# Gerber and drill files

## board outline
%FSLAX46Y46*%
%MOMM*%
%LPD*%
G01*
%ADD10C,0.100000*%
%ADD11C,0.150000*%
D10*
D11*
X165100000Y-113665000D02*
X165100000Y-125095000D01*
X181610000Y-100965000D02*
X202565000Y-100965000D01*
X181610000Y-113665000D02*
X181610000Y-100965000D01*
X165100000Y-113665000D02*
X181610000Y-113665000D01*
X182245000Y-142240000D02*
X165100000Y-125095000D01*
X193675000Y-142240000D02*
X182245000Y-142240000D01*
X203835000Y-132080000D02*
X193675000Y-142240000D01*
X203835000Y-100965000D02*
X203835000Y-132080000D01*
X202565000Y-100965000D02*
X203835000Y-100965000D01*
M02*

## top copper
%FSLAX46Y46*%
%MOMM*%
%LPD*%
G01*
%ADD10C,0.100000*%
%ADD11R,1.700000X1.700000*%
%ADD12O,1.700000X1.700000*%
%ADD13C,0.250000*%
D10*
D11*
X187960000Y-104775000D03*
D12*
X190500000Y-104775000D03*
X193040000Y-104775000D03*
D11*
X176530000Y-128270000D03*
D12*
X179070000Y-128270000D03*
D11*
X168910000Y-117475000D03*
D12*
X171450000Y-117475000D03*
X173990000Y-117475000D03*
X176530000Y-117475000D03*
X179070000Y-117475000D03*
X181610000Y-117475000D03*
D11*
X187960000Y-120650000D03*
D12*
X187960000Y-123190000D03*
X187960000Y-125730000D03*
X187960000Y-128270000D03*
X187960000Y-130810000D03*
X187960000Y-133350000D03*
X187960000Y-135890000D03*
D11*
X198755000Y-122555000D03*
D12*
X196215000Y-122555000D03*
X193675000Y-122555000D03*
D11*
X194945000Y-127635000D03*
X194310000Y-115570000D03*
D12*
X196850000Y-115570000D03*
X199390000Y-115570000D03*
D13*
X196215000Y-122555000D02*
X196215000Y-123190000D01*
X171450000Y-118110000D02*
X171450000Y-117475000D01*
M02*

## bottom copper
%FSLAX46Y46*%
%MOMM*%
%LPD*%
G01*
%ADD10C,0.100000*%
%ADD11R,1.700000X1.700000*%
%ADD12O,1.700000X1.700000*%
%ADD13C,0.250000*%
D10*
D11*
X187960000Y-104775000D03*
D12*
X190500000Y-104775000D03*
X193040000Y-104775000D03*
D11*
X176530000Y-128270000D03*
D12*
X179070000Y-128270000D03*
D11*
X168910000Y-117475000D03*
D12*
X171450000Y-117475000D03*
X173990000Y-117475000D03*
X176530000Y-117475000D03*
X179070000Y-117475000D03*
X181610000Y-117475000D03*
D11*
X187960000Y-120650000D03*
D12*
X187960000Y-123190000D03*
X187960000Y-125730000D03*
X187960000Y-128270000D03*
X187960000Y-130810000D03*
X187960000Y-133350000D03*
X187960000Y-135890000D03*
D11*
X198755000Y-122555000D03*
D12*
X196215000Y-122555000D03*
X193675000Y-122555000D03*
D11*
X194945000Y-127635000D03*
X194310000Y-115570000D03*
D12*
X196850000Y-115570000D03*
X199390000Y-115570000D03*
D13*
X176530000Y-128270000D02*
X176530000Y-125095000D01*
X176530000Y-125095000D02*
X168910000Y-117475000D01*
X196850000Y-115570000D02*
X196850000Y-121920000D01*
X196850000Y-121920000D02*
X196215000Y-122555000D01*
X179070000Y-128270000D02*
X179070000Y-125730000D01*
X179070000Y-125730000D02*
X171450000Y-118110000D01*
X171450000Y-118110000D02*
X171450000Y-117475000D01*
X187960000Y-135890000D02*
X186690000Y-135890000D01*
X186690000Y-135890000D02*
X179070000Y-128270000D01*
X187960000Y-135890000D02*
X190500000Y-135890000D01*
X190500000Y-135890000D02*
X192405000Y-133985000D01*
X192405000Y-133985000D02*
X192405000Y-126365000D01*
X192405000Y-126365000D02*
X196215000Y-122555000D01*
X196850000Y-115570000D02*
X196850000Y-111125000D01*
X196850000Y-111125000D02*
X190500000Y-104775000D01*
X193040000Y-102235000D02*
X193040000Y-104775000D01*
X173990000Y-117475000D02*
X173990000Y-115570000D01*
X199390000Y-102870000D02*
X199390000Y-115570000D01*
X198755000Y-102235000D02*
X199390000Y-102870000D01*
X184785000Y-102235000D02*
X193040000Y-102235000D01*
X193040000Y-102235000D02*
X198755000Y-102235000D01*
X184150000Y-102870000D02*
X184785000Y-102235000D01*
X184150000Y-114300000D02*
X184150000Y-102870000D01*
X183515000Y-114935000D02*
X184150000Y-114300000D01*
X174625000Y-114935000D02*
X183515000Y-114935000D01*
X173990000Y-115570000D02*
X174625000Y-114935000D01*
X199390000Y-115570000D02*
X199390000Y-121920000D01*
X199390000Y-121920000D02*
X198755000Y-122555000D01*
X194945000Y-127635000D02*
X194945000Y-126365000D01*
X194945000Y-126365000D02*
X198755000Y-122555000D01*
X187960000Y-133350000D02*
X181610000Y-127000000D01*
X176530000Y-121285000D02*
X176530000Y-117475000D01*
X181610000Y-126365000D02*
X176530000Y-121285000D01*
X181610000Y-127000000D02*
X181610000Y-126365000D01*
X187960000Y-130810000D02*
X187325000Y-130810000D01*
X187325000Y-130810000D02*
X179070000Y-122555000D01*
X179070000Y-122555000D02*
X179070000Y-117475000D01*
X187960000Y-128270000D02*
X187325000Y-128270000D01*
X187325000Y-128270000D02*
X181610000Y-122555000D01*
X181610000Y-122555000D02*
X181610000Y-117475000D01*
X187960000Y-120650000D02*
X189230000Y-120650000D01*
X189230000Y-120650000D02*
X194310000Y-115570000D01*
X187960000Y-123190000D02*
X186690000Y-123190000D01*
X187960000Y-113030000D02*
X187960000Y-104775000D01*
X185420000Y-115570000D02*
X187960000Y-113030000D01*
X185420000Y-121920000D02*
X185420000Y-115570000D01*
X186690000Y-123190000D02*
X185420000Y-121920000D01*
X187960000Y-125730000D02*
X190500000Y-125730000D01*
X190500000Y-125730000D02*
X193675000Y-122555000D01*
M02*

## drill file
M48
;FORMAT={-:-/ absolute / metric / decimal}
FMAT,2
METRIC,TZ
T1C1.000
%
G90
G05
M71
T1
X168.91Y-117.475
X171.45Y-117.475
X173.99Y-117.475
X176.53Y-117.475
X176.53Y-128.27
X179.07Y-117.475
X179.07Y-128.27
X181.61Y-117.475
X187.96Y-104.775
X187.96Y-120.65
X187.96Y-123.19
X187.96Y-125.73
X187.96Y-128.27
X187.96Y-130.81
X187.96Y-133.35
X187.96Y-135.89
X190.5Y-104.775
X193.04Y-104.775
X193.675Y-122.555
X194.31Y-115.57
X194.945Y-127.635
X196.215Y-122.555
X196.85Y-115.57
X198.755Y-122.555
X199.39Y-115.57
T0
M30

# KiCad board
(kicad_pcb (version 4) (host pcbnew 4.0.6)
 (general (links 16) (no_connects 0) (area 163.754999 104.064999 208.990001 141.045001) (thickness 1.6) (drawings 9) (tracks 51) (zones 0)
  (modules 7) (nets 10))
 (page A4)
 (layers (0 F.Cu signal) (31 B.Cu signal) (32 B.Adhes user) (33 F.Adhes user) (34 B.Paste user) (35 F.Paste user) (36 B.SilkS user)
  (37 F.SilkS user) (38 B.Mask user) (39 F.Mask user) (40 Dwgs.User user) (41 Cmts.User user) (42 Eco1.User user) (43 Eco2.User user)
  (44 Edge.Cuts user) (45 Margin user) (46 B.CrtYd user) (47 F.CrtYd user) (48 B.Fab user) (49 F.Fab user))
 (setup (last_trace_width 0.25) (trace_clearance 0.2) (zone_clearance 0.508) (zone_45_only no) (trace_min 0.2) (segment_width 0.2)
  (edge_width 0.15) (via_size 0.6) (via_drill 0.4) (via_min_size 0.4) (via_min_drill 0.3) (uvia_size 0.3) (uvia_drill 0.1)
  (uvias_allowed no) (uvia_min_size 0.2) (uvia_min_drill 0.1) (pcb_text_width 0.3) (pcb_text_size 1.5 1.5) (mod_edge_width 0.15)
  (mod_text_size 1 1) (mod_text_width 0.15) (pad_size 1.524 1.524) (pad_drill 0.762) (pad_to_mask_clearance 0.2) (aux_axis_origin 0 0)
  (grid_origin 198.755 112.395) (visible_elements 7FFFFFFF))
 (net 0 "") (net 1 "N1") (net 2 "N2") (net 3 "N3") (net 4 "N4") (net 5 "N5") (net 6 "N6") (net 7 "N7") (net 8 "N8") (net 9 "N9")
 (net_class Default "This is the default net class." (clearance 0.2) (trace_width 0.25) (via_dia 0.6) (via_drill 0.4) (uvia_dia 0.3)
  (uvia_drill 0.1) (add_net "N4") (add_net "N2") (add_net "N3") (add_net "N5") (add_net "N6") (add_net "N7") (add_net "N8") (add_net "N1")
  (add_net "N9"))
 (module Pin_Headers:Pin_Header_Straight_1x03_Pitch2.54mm (layer F.Cu) (at 187.96 104.775 90)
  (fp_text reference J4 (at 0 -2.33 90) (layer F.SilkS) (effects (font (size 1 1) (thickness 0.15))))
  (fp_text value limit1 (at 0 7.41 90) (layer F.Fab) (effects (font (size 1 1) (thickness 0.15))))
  (pad 1 thru_hole rect (at 0 0 90) (size 1.7 1.7) (drill 1) (layers *.Cu *.Mask) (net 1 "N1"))
  (pad 2 thru_hole oval (at 0 2.54 90) (size 1.7 1.7) (drill 1) (layers *.Cu *.Mask) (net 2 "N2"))
  (pad 3 thru_hole oval (at 0 5.08 90) (size 1.7 1.7) (drill 1) (layers *.Cu *.Mask) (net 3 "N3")))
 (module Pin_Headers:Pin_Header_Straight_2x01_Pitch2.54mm (layer F.Cu) (at 176.53 128.27)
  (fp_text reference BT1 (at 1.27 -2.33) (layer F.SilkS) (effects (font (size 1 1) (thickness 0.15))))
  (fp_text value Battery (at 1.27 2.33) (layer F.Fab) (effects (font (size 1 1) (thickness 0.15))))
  (pad 1 thru_hole rect (at 0 0) (size 1.7 1.7) (drill 1) (layers *.Cu *.Mask) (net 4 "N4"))
  (pad 2 thru_hole oval (at 2.54 0) (size 1.7 1.7) (drill 1) (layers *.Cu *.Mask) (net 2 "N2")))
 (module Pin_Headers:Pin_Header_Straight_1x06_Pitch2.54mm (layer F.Cu) (at 168.91 117.475 90)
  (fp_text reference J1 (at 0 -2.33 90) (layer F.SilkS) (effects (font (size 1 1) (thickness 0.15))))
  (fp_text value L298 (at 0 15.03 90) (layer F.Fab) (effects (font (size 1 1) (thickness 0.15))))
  (pad 1 thru_hole rect (at 0 0 90) (size 1.7 1.7) (drill 1) (layers *.Cu *.Mask) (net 4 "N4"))
  (pad 2 thru_hole oval (at 0 2.54 90) (size 1.7 1.7) (drill 1) (layers *.Cu *.Mask) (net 2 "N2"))
  (pad 3 thru_hole oval (at 0 5.08 90) (size 1.7 1.7) (drill 1) (layers *.Cu *.Mask) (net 3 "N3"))
  (pad 4 thru_hole oval (at 0 7.62 90) (size 1.7 1.7) (drill 1) (layers *.Cu *.Mask) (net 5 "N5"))
  (pad 5 thru_hole oval (at 0 10.16 90) (size 1.7 1.7) (drill 1) (layers *.Cu *.Mask) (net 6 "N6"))
  (pad 6 thru_hole oval (at 0 12.7 90) (size 1.7 1.7) (drill 1) (layers *.Cu *.Mask) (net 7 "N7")))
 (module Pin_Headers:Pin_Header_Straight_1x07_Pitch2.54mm (layer F.Cu) (at 187.96 120.65)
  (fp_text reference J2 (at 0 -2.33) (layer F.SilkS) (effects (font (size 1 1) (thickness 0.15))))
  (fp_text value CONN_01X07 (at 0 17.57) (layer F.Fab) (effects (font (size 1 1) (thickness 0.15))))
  (pad 1 thru_hole rect (at 0 0) (size 1.7 1.7) (drill 1) (layers *.Cu *.Mask) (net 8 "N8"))
  (pad 2 thru_hole oval (at 0 2.54) (size 1.7 1.7) (drill 1) (layers *.Cu *.Mask) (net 1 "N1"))
  (pad 3 thru_hole oval (at 0 5.08) (size 1.7 1.7) (drill 1) (layers *.Cu *.Mask) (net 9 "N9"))
  (pad 4 thru_hole oval (at 0 7.62) (size 1.7 1.7) (drill 1) (layers *.Cu *.Mask) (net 7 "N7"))
  (pad 5 thru_hole oval (at 0 10.16) (size 1.7 1.7) (drill 1) (layers *.Cu *.Mask) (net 6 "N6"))
  (pad 6 thru_hole oval (at 0 12.7) (size 1.7 1.7) (drill 1) (layers *.Cu *.Mask) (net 5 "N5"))
  (pad 7 thru_hole oval (at 0 15.24) (size 1.7 1.7) (drill 1) (layers *.Cu *.Mask) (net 2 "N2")))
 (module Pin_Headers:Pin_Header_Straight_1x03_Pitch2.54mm (layer F.Cu) (at 198.755 122.555 270)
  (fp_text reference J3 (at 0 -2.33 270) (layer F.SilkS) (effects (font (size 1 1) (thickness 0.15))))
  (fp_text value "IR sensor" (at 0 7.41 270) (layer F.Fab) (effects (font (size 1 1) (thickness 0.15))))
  (pad 1 thru_hole rect (at 0 0 270) (size 1.7 1.7) (drill 1) (layers *.Cu *.Mask) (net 3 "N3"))
  (pad 2 thru_hole oval (at 0 2.54 270) (size 1.7 1.7) (drill 1) (layers *.Cu *.Mask) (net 2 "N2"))
  (pad 3 thru_hole oval (at 0 5.08 270) (size 1.7 1.7) (drill 1) (layers *.Cu *.Mask) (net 9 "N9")))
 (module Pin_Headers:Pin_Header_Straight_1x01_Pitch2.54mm (layer F.Cu) (at 194.945 127.635)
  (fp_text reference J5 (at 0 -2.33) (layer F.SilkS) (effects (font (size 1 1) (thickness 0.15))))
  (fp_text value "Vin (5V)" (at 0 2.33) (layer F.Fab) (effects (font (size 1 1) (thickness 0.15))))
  (pad 1 thru_hole rect (at 0 0) (size 1.7 1.7) (drill 1) (layers *.Cu *.Mask) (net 3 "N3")))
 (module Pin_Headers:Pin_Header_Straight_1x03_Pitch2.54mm (layer F.Cu) (at 194.31 115.57 90)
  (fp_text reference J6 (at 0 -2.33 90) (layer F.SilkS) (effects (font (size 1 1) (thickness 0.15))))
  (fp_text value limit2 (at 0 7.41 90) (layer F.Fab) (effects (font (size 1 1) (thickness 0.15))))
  (pad 1 thru_hole rect (at 0 0 90) (size 1.7 1.7) (drill 1) (layers *.Cu *.Mask) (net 8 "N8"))
  (pad 2 thru_hole oval (at 0 2.54 90) (size 1.7 1.7) (drill 1) (layers *.Cu *.Mask) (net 2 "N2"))
  (pad 3 thru_hole oval (at 0 5.08 90) (size 1.7 1.7) (drill 1) (layers *.Cu *.Mask) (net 3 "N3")))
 (gr_line (start 165.1 113.665) (end 165.1 125.095) (angle 90) (layer Edge.Cuts) (width 0.15))
 (gr_line (start 181.61 100.965) (end 202.565 100.965) (angle 90) (layer Edge.Cuts) (width 0.15))
 (gr_line (start 181.61 113.665) (end 181.61 100.965) (angle 90) (layer Edge.Cuts) (width 0.15))
 (gr_line (start 165.1 113.665) (end 181.61 113.665) (angle 90) (layer Edge.Cuts) (width 0.15))
 (gr_line (start 182.245 142.24) (end 165.1 125.095) (angle 90) (layer Edge.Cuts) (width 0.15))
 (gr_line (start 193.675 142.24) (end 182.245 142.24) (angle 90) (layer Edge.Cuts) (width 0.15))
 (gr_line (start 203.835 132.08) (end 193.675 142.24) (angle 90) (layer Edge.Cuts) (width 0.15))
 (gr_line (start 203.835 100.965) (end 203.835 132.08) (angle 90) (layer Edge.Cuts) (width 0.15))
 (gr_line (start 202.565 100.965) (end 203.835 100.965) (angle 90) (layer Edge.Cuts) (width 0.15))
 (segment (start 176.53 128.27) (end 176.53 125.095) (width 0.25) (layer B.Cu) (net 4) (status 400000))
 (segment (start 176.53 125.095) (end 168.91 117.475) (width 0.25) (layer B.Cu) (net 4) (status 800000))
 (segment (start 196.85 115.57) (end 196.85 121.92) (width 0.25) (layer B.Cu) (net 2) (status 400000))
 (segment (start 196.85 121.92) (end 196.215 122.555) (width 0.25) (layer B.Cu) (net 2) (status 800000))
 (segment (start 179.07 128.27) (end 179.07 125.73) (width 0.25) (layer B.Cu) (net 2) (status 400000))
 (segment (start 179.07 125.73) (end 171.45 118.11) (width 0.25) (layer B.Cu) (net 2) (status 800000))
 (segment (start 171.45 118.11) (end 171.45 117.475) (width 0.25) (layer B.Cu) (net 2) (status C00000))
 (segment (start 187.96 135.89) (end 186.69 135.89) (width 0.25) (layer B.Cu) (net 2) (status 400000))
 (segment (start 186.69 135.89) (end 179.07 128.27) (width 0.25) (layer B.Cu) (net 2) (status 800000))
 (segment (start 187.96 135.89) (end 190.5 135.89) (width 0.25) (layer B.Cu) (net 2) (status 400000))
 (segment (start 190.5 135.89) (end 192.405 133.985) (width 0.25) (layer B.Cu) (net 2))
 (segment (start 192.405 133.985) (end 192.405 126.365) (width 0.25) (layer B.Cu) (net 2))
 (segment (start 192.405 126.365) (end 196.215 122.555) (width 0.25) (layer B.Cu) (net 2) (status 800000))
 (segment (start 196.85 115.57) (end 196.85 111.125) (width 0.25) (layer B.Cu) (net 2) (status 400000))
 (segment (start 196.85 111.125) (end 190.5 104.775) (width 0.25) (layer B.Cu) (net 2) (status 800000))
 (segment (start 196.215 122.555) (end 196.215 123.19) (width 0.25) (layer F.Cu) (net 2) (status C00000))
 (segment (start 171.45 118.11) (end 171.45 117.475) (width 0.25) (layer F.Cu) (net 2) (status 80000))
 (segment (start 193.04 102.235) (end 193.04 104.775) (width 0.25) (layer B.Cu) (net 3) (status 800000))
 (segment (start 173.99 117.475) (end 173.99 115.57) (width 0.25) (layer B.Cu) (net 3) (status 400000))
 (segment (start 199.39 102.87) (end 199.39 115.57) (width 0.25) (layer B.Cu) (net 3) (status 800000))
 (segment (start 198.755 102.235) (end 199.39 102.87) (width 0.25) (layer B.Cu) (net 3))
 (segment (start 184.785 102.235) (end 193.04 102.235) (width 0.25) (layer B.Cu) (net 3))
 (segment (start 193.04 102.235) (end 198.755 102.235) (width 0.25) (layer B.Cu) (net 3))
 (segment (start 184.15 102.87) (end 184.785 102.235) (width 0.25) (layer B.Cu) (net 3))
 (segment (start 184.15 114.3) (end 184.15 102.87) (width 0.25) (layer B.Cu) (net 3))
 (segment (start 183.515 114.935) (end 184.15 114.3) (width 0.25) (layer B.Cu) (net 3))
 (segment (start 174.625 114.935) (end 183.515 114.935) (width 0.25) (layer B.Cu) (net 3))
 (segment (start 173.99 115.57) (end 174.625 114.935) (width 0.25) (layer B.Cu) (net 3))
 (segment (start 199.39 115.57) (end 199.39 121.92) (width 0.25) (layer B.Cu) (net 3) (status C00000))
 (segment (start 199.39 121.92) (end 198.755 122.555) (width 0.25) (layer B.Cu) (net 3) (status C00000))
 (segment (start 194.945 127.635) (end 194.945 126.365) (width 0.25) (layer B.Cu) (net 3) (status 400000))
 (segment (start 194.945 126.365) (end 198.755 122.555) (width 0.25) (layer B.Cu) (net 3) (status 800000))
 (segment (start 187.96 133.35) (end 181.61 127) (width 0.25) (layer B.Cu) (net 5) (status 400000))
 (segment (start 176.53 121.285) (end 176.53 117.475) (width 0.25) (layer B.Cu) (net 5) (status 800000))
 (segment (start 181.61 126.365) (end 176.53 121.285) (width 0.25) (layer B.Cu) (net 5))
 (segment (start 181.61 127) (end 181.61 126.365) (width 0.25) (layer B.Cu) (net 5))
 (segment (start 187.96 130.81) (end 187.325 130.81) (width 0.25) (layer B.Cu) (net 6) (status C00000))
 (segment (start 187.325 130.81) (end 179.07 122.555) (width 0.25) (layer B.Cu) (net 6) (status 400000))
 (segment (start 179.07 122.555) (end 179.07 117.475) (width 0.25) (layer B.Cu) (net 6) (status 800000))
 (segment (start 187.96 128.27) (end 187.325 128.27) (width 0.25) (layer B.Cu) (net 7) (status C00000))
 (segment (start 187.325 128.27) (end 181.61 122.555) (width 0.25) (layer B.Cu) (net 7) (status 400000))
 (segment (start 181.61 122.555) (end 181.61 117.475) (width 0.25) (layer B.Cu) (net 7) (status 800000))
 (segment (start 187.96 120.65) (end 189.23 120.65) (width 0.25) (layer B.Cu) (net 8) (status 400000))
 (segment (start 189.23 120.65) (end 194.31 115.57) (width 0.25) (layer B.Cu) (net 8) (status 800000))
 (segment (start 187.96 123.19) (end 186.69 123.19) (width 0.25) (layer B.Cu) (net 1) (status 400000))
 (segment (start 187.96 113.03) (end 187.96 104.775) (width 0.25) (layer B.Cu) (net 1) (status 800000))
 (segment (start 185.42 115.57) (end 187.96 113.03) (width 0.25) (layer B.Cu) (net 1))
 (segment (start 185.42 121.92) (end 185.42 115.57) (width 0.25) (layer B.Cu) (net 1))
 (segment (start 186.69 123.19) (end 185.42 121.92) (width 0.25) (layer B.Cu) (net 1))
 (segment (start 187.96 125.73) (end 190.5 125.73) (width 0.25) (layer B.Cu) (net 9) (status 400000))
 (segment (start 190.5 125.73) (end 193.675 122.555) (width 0.25) (layer B.Cu) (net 9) (status 800000)))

